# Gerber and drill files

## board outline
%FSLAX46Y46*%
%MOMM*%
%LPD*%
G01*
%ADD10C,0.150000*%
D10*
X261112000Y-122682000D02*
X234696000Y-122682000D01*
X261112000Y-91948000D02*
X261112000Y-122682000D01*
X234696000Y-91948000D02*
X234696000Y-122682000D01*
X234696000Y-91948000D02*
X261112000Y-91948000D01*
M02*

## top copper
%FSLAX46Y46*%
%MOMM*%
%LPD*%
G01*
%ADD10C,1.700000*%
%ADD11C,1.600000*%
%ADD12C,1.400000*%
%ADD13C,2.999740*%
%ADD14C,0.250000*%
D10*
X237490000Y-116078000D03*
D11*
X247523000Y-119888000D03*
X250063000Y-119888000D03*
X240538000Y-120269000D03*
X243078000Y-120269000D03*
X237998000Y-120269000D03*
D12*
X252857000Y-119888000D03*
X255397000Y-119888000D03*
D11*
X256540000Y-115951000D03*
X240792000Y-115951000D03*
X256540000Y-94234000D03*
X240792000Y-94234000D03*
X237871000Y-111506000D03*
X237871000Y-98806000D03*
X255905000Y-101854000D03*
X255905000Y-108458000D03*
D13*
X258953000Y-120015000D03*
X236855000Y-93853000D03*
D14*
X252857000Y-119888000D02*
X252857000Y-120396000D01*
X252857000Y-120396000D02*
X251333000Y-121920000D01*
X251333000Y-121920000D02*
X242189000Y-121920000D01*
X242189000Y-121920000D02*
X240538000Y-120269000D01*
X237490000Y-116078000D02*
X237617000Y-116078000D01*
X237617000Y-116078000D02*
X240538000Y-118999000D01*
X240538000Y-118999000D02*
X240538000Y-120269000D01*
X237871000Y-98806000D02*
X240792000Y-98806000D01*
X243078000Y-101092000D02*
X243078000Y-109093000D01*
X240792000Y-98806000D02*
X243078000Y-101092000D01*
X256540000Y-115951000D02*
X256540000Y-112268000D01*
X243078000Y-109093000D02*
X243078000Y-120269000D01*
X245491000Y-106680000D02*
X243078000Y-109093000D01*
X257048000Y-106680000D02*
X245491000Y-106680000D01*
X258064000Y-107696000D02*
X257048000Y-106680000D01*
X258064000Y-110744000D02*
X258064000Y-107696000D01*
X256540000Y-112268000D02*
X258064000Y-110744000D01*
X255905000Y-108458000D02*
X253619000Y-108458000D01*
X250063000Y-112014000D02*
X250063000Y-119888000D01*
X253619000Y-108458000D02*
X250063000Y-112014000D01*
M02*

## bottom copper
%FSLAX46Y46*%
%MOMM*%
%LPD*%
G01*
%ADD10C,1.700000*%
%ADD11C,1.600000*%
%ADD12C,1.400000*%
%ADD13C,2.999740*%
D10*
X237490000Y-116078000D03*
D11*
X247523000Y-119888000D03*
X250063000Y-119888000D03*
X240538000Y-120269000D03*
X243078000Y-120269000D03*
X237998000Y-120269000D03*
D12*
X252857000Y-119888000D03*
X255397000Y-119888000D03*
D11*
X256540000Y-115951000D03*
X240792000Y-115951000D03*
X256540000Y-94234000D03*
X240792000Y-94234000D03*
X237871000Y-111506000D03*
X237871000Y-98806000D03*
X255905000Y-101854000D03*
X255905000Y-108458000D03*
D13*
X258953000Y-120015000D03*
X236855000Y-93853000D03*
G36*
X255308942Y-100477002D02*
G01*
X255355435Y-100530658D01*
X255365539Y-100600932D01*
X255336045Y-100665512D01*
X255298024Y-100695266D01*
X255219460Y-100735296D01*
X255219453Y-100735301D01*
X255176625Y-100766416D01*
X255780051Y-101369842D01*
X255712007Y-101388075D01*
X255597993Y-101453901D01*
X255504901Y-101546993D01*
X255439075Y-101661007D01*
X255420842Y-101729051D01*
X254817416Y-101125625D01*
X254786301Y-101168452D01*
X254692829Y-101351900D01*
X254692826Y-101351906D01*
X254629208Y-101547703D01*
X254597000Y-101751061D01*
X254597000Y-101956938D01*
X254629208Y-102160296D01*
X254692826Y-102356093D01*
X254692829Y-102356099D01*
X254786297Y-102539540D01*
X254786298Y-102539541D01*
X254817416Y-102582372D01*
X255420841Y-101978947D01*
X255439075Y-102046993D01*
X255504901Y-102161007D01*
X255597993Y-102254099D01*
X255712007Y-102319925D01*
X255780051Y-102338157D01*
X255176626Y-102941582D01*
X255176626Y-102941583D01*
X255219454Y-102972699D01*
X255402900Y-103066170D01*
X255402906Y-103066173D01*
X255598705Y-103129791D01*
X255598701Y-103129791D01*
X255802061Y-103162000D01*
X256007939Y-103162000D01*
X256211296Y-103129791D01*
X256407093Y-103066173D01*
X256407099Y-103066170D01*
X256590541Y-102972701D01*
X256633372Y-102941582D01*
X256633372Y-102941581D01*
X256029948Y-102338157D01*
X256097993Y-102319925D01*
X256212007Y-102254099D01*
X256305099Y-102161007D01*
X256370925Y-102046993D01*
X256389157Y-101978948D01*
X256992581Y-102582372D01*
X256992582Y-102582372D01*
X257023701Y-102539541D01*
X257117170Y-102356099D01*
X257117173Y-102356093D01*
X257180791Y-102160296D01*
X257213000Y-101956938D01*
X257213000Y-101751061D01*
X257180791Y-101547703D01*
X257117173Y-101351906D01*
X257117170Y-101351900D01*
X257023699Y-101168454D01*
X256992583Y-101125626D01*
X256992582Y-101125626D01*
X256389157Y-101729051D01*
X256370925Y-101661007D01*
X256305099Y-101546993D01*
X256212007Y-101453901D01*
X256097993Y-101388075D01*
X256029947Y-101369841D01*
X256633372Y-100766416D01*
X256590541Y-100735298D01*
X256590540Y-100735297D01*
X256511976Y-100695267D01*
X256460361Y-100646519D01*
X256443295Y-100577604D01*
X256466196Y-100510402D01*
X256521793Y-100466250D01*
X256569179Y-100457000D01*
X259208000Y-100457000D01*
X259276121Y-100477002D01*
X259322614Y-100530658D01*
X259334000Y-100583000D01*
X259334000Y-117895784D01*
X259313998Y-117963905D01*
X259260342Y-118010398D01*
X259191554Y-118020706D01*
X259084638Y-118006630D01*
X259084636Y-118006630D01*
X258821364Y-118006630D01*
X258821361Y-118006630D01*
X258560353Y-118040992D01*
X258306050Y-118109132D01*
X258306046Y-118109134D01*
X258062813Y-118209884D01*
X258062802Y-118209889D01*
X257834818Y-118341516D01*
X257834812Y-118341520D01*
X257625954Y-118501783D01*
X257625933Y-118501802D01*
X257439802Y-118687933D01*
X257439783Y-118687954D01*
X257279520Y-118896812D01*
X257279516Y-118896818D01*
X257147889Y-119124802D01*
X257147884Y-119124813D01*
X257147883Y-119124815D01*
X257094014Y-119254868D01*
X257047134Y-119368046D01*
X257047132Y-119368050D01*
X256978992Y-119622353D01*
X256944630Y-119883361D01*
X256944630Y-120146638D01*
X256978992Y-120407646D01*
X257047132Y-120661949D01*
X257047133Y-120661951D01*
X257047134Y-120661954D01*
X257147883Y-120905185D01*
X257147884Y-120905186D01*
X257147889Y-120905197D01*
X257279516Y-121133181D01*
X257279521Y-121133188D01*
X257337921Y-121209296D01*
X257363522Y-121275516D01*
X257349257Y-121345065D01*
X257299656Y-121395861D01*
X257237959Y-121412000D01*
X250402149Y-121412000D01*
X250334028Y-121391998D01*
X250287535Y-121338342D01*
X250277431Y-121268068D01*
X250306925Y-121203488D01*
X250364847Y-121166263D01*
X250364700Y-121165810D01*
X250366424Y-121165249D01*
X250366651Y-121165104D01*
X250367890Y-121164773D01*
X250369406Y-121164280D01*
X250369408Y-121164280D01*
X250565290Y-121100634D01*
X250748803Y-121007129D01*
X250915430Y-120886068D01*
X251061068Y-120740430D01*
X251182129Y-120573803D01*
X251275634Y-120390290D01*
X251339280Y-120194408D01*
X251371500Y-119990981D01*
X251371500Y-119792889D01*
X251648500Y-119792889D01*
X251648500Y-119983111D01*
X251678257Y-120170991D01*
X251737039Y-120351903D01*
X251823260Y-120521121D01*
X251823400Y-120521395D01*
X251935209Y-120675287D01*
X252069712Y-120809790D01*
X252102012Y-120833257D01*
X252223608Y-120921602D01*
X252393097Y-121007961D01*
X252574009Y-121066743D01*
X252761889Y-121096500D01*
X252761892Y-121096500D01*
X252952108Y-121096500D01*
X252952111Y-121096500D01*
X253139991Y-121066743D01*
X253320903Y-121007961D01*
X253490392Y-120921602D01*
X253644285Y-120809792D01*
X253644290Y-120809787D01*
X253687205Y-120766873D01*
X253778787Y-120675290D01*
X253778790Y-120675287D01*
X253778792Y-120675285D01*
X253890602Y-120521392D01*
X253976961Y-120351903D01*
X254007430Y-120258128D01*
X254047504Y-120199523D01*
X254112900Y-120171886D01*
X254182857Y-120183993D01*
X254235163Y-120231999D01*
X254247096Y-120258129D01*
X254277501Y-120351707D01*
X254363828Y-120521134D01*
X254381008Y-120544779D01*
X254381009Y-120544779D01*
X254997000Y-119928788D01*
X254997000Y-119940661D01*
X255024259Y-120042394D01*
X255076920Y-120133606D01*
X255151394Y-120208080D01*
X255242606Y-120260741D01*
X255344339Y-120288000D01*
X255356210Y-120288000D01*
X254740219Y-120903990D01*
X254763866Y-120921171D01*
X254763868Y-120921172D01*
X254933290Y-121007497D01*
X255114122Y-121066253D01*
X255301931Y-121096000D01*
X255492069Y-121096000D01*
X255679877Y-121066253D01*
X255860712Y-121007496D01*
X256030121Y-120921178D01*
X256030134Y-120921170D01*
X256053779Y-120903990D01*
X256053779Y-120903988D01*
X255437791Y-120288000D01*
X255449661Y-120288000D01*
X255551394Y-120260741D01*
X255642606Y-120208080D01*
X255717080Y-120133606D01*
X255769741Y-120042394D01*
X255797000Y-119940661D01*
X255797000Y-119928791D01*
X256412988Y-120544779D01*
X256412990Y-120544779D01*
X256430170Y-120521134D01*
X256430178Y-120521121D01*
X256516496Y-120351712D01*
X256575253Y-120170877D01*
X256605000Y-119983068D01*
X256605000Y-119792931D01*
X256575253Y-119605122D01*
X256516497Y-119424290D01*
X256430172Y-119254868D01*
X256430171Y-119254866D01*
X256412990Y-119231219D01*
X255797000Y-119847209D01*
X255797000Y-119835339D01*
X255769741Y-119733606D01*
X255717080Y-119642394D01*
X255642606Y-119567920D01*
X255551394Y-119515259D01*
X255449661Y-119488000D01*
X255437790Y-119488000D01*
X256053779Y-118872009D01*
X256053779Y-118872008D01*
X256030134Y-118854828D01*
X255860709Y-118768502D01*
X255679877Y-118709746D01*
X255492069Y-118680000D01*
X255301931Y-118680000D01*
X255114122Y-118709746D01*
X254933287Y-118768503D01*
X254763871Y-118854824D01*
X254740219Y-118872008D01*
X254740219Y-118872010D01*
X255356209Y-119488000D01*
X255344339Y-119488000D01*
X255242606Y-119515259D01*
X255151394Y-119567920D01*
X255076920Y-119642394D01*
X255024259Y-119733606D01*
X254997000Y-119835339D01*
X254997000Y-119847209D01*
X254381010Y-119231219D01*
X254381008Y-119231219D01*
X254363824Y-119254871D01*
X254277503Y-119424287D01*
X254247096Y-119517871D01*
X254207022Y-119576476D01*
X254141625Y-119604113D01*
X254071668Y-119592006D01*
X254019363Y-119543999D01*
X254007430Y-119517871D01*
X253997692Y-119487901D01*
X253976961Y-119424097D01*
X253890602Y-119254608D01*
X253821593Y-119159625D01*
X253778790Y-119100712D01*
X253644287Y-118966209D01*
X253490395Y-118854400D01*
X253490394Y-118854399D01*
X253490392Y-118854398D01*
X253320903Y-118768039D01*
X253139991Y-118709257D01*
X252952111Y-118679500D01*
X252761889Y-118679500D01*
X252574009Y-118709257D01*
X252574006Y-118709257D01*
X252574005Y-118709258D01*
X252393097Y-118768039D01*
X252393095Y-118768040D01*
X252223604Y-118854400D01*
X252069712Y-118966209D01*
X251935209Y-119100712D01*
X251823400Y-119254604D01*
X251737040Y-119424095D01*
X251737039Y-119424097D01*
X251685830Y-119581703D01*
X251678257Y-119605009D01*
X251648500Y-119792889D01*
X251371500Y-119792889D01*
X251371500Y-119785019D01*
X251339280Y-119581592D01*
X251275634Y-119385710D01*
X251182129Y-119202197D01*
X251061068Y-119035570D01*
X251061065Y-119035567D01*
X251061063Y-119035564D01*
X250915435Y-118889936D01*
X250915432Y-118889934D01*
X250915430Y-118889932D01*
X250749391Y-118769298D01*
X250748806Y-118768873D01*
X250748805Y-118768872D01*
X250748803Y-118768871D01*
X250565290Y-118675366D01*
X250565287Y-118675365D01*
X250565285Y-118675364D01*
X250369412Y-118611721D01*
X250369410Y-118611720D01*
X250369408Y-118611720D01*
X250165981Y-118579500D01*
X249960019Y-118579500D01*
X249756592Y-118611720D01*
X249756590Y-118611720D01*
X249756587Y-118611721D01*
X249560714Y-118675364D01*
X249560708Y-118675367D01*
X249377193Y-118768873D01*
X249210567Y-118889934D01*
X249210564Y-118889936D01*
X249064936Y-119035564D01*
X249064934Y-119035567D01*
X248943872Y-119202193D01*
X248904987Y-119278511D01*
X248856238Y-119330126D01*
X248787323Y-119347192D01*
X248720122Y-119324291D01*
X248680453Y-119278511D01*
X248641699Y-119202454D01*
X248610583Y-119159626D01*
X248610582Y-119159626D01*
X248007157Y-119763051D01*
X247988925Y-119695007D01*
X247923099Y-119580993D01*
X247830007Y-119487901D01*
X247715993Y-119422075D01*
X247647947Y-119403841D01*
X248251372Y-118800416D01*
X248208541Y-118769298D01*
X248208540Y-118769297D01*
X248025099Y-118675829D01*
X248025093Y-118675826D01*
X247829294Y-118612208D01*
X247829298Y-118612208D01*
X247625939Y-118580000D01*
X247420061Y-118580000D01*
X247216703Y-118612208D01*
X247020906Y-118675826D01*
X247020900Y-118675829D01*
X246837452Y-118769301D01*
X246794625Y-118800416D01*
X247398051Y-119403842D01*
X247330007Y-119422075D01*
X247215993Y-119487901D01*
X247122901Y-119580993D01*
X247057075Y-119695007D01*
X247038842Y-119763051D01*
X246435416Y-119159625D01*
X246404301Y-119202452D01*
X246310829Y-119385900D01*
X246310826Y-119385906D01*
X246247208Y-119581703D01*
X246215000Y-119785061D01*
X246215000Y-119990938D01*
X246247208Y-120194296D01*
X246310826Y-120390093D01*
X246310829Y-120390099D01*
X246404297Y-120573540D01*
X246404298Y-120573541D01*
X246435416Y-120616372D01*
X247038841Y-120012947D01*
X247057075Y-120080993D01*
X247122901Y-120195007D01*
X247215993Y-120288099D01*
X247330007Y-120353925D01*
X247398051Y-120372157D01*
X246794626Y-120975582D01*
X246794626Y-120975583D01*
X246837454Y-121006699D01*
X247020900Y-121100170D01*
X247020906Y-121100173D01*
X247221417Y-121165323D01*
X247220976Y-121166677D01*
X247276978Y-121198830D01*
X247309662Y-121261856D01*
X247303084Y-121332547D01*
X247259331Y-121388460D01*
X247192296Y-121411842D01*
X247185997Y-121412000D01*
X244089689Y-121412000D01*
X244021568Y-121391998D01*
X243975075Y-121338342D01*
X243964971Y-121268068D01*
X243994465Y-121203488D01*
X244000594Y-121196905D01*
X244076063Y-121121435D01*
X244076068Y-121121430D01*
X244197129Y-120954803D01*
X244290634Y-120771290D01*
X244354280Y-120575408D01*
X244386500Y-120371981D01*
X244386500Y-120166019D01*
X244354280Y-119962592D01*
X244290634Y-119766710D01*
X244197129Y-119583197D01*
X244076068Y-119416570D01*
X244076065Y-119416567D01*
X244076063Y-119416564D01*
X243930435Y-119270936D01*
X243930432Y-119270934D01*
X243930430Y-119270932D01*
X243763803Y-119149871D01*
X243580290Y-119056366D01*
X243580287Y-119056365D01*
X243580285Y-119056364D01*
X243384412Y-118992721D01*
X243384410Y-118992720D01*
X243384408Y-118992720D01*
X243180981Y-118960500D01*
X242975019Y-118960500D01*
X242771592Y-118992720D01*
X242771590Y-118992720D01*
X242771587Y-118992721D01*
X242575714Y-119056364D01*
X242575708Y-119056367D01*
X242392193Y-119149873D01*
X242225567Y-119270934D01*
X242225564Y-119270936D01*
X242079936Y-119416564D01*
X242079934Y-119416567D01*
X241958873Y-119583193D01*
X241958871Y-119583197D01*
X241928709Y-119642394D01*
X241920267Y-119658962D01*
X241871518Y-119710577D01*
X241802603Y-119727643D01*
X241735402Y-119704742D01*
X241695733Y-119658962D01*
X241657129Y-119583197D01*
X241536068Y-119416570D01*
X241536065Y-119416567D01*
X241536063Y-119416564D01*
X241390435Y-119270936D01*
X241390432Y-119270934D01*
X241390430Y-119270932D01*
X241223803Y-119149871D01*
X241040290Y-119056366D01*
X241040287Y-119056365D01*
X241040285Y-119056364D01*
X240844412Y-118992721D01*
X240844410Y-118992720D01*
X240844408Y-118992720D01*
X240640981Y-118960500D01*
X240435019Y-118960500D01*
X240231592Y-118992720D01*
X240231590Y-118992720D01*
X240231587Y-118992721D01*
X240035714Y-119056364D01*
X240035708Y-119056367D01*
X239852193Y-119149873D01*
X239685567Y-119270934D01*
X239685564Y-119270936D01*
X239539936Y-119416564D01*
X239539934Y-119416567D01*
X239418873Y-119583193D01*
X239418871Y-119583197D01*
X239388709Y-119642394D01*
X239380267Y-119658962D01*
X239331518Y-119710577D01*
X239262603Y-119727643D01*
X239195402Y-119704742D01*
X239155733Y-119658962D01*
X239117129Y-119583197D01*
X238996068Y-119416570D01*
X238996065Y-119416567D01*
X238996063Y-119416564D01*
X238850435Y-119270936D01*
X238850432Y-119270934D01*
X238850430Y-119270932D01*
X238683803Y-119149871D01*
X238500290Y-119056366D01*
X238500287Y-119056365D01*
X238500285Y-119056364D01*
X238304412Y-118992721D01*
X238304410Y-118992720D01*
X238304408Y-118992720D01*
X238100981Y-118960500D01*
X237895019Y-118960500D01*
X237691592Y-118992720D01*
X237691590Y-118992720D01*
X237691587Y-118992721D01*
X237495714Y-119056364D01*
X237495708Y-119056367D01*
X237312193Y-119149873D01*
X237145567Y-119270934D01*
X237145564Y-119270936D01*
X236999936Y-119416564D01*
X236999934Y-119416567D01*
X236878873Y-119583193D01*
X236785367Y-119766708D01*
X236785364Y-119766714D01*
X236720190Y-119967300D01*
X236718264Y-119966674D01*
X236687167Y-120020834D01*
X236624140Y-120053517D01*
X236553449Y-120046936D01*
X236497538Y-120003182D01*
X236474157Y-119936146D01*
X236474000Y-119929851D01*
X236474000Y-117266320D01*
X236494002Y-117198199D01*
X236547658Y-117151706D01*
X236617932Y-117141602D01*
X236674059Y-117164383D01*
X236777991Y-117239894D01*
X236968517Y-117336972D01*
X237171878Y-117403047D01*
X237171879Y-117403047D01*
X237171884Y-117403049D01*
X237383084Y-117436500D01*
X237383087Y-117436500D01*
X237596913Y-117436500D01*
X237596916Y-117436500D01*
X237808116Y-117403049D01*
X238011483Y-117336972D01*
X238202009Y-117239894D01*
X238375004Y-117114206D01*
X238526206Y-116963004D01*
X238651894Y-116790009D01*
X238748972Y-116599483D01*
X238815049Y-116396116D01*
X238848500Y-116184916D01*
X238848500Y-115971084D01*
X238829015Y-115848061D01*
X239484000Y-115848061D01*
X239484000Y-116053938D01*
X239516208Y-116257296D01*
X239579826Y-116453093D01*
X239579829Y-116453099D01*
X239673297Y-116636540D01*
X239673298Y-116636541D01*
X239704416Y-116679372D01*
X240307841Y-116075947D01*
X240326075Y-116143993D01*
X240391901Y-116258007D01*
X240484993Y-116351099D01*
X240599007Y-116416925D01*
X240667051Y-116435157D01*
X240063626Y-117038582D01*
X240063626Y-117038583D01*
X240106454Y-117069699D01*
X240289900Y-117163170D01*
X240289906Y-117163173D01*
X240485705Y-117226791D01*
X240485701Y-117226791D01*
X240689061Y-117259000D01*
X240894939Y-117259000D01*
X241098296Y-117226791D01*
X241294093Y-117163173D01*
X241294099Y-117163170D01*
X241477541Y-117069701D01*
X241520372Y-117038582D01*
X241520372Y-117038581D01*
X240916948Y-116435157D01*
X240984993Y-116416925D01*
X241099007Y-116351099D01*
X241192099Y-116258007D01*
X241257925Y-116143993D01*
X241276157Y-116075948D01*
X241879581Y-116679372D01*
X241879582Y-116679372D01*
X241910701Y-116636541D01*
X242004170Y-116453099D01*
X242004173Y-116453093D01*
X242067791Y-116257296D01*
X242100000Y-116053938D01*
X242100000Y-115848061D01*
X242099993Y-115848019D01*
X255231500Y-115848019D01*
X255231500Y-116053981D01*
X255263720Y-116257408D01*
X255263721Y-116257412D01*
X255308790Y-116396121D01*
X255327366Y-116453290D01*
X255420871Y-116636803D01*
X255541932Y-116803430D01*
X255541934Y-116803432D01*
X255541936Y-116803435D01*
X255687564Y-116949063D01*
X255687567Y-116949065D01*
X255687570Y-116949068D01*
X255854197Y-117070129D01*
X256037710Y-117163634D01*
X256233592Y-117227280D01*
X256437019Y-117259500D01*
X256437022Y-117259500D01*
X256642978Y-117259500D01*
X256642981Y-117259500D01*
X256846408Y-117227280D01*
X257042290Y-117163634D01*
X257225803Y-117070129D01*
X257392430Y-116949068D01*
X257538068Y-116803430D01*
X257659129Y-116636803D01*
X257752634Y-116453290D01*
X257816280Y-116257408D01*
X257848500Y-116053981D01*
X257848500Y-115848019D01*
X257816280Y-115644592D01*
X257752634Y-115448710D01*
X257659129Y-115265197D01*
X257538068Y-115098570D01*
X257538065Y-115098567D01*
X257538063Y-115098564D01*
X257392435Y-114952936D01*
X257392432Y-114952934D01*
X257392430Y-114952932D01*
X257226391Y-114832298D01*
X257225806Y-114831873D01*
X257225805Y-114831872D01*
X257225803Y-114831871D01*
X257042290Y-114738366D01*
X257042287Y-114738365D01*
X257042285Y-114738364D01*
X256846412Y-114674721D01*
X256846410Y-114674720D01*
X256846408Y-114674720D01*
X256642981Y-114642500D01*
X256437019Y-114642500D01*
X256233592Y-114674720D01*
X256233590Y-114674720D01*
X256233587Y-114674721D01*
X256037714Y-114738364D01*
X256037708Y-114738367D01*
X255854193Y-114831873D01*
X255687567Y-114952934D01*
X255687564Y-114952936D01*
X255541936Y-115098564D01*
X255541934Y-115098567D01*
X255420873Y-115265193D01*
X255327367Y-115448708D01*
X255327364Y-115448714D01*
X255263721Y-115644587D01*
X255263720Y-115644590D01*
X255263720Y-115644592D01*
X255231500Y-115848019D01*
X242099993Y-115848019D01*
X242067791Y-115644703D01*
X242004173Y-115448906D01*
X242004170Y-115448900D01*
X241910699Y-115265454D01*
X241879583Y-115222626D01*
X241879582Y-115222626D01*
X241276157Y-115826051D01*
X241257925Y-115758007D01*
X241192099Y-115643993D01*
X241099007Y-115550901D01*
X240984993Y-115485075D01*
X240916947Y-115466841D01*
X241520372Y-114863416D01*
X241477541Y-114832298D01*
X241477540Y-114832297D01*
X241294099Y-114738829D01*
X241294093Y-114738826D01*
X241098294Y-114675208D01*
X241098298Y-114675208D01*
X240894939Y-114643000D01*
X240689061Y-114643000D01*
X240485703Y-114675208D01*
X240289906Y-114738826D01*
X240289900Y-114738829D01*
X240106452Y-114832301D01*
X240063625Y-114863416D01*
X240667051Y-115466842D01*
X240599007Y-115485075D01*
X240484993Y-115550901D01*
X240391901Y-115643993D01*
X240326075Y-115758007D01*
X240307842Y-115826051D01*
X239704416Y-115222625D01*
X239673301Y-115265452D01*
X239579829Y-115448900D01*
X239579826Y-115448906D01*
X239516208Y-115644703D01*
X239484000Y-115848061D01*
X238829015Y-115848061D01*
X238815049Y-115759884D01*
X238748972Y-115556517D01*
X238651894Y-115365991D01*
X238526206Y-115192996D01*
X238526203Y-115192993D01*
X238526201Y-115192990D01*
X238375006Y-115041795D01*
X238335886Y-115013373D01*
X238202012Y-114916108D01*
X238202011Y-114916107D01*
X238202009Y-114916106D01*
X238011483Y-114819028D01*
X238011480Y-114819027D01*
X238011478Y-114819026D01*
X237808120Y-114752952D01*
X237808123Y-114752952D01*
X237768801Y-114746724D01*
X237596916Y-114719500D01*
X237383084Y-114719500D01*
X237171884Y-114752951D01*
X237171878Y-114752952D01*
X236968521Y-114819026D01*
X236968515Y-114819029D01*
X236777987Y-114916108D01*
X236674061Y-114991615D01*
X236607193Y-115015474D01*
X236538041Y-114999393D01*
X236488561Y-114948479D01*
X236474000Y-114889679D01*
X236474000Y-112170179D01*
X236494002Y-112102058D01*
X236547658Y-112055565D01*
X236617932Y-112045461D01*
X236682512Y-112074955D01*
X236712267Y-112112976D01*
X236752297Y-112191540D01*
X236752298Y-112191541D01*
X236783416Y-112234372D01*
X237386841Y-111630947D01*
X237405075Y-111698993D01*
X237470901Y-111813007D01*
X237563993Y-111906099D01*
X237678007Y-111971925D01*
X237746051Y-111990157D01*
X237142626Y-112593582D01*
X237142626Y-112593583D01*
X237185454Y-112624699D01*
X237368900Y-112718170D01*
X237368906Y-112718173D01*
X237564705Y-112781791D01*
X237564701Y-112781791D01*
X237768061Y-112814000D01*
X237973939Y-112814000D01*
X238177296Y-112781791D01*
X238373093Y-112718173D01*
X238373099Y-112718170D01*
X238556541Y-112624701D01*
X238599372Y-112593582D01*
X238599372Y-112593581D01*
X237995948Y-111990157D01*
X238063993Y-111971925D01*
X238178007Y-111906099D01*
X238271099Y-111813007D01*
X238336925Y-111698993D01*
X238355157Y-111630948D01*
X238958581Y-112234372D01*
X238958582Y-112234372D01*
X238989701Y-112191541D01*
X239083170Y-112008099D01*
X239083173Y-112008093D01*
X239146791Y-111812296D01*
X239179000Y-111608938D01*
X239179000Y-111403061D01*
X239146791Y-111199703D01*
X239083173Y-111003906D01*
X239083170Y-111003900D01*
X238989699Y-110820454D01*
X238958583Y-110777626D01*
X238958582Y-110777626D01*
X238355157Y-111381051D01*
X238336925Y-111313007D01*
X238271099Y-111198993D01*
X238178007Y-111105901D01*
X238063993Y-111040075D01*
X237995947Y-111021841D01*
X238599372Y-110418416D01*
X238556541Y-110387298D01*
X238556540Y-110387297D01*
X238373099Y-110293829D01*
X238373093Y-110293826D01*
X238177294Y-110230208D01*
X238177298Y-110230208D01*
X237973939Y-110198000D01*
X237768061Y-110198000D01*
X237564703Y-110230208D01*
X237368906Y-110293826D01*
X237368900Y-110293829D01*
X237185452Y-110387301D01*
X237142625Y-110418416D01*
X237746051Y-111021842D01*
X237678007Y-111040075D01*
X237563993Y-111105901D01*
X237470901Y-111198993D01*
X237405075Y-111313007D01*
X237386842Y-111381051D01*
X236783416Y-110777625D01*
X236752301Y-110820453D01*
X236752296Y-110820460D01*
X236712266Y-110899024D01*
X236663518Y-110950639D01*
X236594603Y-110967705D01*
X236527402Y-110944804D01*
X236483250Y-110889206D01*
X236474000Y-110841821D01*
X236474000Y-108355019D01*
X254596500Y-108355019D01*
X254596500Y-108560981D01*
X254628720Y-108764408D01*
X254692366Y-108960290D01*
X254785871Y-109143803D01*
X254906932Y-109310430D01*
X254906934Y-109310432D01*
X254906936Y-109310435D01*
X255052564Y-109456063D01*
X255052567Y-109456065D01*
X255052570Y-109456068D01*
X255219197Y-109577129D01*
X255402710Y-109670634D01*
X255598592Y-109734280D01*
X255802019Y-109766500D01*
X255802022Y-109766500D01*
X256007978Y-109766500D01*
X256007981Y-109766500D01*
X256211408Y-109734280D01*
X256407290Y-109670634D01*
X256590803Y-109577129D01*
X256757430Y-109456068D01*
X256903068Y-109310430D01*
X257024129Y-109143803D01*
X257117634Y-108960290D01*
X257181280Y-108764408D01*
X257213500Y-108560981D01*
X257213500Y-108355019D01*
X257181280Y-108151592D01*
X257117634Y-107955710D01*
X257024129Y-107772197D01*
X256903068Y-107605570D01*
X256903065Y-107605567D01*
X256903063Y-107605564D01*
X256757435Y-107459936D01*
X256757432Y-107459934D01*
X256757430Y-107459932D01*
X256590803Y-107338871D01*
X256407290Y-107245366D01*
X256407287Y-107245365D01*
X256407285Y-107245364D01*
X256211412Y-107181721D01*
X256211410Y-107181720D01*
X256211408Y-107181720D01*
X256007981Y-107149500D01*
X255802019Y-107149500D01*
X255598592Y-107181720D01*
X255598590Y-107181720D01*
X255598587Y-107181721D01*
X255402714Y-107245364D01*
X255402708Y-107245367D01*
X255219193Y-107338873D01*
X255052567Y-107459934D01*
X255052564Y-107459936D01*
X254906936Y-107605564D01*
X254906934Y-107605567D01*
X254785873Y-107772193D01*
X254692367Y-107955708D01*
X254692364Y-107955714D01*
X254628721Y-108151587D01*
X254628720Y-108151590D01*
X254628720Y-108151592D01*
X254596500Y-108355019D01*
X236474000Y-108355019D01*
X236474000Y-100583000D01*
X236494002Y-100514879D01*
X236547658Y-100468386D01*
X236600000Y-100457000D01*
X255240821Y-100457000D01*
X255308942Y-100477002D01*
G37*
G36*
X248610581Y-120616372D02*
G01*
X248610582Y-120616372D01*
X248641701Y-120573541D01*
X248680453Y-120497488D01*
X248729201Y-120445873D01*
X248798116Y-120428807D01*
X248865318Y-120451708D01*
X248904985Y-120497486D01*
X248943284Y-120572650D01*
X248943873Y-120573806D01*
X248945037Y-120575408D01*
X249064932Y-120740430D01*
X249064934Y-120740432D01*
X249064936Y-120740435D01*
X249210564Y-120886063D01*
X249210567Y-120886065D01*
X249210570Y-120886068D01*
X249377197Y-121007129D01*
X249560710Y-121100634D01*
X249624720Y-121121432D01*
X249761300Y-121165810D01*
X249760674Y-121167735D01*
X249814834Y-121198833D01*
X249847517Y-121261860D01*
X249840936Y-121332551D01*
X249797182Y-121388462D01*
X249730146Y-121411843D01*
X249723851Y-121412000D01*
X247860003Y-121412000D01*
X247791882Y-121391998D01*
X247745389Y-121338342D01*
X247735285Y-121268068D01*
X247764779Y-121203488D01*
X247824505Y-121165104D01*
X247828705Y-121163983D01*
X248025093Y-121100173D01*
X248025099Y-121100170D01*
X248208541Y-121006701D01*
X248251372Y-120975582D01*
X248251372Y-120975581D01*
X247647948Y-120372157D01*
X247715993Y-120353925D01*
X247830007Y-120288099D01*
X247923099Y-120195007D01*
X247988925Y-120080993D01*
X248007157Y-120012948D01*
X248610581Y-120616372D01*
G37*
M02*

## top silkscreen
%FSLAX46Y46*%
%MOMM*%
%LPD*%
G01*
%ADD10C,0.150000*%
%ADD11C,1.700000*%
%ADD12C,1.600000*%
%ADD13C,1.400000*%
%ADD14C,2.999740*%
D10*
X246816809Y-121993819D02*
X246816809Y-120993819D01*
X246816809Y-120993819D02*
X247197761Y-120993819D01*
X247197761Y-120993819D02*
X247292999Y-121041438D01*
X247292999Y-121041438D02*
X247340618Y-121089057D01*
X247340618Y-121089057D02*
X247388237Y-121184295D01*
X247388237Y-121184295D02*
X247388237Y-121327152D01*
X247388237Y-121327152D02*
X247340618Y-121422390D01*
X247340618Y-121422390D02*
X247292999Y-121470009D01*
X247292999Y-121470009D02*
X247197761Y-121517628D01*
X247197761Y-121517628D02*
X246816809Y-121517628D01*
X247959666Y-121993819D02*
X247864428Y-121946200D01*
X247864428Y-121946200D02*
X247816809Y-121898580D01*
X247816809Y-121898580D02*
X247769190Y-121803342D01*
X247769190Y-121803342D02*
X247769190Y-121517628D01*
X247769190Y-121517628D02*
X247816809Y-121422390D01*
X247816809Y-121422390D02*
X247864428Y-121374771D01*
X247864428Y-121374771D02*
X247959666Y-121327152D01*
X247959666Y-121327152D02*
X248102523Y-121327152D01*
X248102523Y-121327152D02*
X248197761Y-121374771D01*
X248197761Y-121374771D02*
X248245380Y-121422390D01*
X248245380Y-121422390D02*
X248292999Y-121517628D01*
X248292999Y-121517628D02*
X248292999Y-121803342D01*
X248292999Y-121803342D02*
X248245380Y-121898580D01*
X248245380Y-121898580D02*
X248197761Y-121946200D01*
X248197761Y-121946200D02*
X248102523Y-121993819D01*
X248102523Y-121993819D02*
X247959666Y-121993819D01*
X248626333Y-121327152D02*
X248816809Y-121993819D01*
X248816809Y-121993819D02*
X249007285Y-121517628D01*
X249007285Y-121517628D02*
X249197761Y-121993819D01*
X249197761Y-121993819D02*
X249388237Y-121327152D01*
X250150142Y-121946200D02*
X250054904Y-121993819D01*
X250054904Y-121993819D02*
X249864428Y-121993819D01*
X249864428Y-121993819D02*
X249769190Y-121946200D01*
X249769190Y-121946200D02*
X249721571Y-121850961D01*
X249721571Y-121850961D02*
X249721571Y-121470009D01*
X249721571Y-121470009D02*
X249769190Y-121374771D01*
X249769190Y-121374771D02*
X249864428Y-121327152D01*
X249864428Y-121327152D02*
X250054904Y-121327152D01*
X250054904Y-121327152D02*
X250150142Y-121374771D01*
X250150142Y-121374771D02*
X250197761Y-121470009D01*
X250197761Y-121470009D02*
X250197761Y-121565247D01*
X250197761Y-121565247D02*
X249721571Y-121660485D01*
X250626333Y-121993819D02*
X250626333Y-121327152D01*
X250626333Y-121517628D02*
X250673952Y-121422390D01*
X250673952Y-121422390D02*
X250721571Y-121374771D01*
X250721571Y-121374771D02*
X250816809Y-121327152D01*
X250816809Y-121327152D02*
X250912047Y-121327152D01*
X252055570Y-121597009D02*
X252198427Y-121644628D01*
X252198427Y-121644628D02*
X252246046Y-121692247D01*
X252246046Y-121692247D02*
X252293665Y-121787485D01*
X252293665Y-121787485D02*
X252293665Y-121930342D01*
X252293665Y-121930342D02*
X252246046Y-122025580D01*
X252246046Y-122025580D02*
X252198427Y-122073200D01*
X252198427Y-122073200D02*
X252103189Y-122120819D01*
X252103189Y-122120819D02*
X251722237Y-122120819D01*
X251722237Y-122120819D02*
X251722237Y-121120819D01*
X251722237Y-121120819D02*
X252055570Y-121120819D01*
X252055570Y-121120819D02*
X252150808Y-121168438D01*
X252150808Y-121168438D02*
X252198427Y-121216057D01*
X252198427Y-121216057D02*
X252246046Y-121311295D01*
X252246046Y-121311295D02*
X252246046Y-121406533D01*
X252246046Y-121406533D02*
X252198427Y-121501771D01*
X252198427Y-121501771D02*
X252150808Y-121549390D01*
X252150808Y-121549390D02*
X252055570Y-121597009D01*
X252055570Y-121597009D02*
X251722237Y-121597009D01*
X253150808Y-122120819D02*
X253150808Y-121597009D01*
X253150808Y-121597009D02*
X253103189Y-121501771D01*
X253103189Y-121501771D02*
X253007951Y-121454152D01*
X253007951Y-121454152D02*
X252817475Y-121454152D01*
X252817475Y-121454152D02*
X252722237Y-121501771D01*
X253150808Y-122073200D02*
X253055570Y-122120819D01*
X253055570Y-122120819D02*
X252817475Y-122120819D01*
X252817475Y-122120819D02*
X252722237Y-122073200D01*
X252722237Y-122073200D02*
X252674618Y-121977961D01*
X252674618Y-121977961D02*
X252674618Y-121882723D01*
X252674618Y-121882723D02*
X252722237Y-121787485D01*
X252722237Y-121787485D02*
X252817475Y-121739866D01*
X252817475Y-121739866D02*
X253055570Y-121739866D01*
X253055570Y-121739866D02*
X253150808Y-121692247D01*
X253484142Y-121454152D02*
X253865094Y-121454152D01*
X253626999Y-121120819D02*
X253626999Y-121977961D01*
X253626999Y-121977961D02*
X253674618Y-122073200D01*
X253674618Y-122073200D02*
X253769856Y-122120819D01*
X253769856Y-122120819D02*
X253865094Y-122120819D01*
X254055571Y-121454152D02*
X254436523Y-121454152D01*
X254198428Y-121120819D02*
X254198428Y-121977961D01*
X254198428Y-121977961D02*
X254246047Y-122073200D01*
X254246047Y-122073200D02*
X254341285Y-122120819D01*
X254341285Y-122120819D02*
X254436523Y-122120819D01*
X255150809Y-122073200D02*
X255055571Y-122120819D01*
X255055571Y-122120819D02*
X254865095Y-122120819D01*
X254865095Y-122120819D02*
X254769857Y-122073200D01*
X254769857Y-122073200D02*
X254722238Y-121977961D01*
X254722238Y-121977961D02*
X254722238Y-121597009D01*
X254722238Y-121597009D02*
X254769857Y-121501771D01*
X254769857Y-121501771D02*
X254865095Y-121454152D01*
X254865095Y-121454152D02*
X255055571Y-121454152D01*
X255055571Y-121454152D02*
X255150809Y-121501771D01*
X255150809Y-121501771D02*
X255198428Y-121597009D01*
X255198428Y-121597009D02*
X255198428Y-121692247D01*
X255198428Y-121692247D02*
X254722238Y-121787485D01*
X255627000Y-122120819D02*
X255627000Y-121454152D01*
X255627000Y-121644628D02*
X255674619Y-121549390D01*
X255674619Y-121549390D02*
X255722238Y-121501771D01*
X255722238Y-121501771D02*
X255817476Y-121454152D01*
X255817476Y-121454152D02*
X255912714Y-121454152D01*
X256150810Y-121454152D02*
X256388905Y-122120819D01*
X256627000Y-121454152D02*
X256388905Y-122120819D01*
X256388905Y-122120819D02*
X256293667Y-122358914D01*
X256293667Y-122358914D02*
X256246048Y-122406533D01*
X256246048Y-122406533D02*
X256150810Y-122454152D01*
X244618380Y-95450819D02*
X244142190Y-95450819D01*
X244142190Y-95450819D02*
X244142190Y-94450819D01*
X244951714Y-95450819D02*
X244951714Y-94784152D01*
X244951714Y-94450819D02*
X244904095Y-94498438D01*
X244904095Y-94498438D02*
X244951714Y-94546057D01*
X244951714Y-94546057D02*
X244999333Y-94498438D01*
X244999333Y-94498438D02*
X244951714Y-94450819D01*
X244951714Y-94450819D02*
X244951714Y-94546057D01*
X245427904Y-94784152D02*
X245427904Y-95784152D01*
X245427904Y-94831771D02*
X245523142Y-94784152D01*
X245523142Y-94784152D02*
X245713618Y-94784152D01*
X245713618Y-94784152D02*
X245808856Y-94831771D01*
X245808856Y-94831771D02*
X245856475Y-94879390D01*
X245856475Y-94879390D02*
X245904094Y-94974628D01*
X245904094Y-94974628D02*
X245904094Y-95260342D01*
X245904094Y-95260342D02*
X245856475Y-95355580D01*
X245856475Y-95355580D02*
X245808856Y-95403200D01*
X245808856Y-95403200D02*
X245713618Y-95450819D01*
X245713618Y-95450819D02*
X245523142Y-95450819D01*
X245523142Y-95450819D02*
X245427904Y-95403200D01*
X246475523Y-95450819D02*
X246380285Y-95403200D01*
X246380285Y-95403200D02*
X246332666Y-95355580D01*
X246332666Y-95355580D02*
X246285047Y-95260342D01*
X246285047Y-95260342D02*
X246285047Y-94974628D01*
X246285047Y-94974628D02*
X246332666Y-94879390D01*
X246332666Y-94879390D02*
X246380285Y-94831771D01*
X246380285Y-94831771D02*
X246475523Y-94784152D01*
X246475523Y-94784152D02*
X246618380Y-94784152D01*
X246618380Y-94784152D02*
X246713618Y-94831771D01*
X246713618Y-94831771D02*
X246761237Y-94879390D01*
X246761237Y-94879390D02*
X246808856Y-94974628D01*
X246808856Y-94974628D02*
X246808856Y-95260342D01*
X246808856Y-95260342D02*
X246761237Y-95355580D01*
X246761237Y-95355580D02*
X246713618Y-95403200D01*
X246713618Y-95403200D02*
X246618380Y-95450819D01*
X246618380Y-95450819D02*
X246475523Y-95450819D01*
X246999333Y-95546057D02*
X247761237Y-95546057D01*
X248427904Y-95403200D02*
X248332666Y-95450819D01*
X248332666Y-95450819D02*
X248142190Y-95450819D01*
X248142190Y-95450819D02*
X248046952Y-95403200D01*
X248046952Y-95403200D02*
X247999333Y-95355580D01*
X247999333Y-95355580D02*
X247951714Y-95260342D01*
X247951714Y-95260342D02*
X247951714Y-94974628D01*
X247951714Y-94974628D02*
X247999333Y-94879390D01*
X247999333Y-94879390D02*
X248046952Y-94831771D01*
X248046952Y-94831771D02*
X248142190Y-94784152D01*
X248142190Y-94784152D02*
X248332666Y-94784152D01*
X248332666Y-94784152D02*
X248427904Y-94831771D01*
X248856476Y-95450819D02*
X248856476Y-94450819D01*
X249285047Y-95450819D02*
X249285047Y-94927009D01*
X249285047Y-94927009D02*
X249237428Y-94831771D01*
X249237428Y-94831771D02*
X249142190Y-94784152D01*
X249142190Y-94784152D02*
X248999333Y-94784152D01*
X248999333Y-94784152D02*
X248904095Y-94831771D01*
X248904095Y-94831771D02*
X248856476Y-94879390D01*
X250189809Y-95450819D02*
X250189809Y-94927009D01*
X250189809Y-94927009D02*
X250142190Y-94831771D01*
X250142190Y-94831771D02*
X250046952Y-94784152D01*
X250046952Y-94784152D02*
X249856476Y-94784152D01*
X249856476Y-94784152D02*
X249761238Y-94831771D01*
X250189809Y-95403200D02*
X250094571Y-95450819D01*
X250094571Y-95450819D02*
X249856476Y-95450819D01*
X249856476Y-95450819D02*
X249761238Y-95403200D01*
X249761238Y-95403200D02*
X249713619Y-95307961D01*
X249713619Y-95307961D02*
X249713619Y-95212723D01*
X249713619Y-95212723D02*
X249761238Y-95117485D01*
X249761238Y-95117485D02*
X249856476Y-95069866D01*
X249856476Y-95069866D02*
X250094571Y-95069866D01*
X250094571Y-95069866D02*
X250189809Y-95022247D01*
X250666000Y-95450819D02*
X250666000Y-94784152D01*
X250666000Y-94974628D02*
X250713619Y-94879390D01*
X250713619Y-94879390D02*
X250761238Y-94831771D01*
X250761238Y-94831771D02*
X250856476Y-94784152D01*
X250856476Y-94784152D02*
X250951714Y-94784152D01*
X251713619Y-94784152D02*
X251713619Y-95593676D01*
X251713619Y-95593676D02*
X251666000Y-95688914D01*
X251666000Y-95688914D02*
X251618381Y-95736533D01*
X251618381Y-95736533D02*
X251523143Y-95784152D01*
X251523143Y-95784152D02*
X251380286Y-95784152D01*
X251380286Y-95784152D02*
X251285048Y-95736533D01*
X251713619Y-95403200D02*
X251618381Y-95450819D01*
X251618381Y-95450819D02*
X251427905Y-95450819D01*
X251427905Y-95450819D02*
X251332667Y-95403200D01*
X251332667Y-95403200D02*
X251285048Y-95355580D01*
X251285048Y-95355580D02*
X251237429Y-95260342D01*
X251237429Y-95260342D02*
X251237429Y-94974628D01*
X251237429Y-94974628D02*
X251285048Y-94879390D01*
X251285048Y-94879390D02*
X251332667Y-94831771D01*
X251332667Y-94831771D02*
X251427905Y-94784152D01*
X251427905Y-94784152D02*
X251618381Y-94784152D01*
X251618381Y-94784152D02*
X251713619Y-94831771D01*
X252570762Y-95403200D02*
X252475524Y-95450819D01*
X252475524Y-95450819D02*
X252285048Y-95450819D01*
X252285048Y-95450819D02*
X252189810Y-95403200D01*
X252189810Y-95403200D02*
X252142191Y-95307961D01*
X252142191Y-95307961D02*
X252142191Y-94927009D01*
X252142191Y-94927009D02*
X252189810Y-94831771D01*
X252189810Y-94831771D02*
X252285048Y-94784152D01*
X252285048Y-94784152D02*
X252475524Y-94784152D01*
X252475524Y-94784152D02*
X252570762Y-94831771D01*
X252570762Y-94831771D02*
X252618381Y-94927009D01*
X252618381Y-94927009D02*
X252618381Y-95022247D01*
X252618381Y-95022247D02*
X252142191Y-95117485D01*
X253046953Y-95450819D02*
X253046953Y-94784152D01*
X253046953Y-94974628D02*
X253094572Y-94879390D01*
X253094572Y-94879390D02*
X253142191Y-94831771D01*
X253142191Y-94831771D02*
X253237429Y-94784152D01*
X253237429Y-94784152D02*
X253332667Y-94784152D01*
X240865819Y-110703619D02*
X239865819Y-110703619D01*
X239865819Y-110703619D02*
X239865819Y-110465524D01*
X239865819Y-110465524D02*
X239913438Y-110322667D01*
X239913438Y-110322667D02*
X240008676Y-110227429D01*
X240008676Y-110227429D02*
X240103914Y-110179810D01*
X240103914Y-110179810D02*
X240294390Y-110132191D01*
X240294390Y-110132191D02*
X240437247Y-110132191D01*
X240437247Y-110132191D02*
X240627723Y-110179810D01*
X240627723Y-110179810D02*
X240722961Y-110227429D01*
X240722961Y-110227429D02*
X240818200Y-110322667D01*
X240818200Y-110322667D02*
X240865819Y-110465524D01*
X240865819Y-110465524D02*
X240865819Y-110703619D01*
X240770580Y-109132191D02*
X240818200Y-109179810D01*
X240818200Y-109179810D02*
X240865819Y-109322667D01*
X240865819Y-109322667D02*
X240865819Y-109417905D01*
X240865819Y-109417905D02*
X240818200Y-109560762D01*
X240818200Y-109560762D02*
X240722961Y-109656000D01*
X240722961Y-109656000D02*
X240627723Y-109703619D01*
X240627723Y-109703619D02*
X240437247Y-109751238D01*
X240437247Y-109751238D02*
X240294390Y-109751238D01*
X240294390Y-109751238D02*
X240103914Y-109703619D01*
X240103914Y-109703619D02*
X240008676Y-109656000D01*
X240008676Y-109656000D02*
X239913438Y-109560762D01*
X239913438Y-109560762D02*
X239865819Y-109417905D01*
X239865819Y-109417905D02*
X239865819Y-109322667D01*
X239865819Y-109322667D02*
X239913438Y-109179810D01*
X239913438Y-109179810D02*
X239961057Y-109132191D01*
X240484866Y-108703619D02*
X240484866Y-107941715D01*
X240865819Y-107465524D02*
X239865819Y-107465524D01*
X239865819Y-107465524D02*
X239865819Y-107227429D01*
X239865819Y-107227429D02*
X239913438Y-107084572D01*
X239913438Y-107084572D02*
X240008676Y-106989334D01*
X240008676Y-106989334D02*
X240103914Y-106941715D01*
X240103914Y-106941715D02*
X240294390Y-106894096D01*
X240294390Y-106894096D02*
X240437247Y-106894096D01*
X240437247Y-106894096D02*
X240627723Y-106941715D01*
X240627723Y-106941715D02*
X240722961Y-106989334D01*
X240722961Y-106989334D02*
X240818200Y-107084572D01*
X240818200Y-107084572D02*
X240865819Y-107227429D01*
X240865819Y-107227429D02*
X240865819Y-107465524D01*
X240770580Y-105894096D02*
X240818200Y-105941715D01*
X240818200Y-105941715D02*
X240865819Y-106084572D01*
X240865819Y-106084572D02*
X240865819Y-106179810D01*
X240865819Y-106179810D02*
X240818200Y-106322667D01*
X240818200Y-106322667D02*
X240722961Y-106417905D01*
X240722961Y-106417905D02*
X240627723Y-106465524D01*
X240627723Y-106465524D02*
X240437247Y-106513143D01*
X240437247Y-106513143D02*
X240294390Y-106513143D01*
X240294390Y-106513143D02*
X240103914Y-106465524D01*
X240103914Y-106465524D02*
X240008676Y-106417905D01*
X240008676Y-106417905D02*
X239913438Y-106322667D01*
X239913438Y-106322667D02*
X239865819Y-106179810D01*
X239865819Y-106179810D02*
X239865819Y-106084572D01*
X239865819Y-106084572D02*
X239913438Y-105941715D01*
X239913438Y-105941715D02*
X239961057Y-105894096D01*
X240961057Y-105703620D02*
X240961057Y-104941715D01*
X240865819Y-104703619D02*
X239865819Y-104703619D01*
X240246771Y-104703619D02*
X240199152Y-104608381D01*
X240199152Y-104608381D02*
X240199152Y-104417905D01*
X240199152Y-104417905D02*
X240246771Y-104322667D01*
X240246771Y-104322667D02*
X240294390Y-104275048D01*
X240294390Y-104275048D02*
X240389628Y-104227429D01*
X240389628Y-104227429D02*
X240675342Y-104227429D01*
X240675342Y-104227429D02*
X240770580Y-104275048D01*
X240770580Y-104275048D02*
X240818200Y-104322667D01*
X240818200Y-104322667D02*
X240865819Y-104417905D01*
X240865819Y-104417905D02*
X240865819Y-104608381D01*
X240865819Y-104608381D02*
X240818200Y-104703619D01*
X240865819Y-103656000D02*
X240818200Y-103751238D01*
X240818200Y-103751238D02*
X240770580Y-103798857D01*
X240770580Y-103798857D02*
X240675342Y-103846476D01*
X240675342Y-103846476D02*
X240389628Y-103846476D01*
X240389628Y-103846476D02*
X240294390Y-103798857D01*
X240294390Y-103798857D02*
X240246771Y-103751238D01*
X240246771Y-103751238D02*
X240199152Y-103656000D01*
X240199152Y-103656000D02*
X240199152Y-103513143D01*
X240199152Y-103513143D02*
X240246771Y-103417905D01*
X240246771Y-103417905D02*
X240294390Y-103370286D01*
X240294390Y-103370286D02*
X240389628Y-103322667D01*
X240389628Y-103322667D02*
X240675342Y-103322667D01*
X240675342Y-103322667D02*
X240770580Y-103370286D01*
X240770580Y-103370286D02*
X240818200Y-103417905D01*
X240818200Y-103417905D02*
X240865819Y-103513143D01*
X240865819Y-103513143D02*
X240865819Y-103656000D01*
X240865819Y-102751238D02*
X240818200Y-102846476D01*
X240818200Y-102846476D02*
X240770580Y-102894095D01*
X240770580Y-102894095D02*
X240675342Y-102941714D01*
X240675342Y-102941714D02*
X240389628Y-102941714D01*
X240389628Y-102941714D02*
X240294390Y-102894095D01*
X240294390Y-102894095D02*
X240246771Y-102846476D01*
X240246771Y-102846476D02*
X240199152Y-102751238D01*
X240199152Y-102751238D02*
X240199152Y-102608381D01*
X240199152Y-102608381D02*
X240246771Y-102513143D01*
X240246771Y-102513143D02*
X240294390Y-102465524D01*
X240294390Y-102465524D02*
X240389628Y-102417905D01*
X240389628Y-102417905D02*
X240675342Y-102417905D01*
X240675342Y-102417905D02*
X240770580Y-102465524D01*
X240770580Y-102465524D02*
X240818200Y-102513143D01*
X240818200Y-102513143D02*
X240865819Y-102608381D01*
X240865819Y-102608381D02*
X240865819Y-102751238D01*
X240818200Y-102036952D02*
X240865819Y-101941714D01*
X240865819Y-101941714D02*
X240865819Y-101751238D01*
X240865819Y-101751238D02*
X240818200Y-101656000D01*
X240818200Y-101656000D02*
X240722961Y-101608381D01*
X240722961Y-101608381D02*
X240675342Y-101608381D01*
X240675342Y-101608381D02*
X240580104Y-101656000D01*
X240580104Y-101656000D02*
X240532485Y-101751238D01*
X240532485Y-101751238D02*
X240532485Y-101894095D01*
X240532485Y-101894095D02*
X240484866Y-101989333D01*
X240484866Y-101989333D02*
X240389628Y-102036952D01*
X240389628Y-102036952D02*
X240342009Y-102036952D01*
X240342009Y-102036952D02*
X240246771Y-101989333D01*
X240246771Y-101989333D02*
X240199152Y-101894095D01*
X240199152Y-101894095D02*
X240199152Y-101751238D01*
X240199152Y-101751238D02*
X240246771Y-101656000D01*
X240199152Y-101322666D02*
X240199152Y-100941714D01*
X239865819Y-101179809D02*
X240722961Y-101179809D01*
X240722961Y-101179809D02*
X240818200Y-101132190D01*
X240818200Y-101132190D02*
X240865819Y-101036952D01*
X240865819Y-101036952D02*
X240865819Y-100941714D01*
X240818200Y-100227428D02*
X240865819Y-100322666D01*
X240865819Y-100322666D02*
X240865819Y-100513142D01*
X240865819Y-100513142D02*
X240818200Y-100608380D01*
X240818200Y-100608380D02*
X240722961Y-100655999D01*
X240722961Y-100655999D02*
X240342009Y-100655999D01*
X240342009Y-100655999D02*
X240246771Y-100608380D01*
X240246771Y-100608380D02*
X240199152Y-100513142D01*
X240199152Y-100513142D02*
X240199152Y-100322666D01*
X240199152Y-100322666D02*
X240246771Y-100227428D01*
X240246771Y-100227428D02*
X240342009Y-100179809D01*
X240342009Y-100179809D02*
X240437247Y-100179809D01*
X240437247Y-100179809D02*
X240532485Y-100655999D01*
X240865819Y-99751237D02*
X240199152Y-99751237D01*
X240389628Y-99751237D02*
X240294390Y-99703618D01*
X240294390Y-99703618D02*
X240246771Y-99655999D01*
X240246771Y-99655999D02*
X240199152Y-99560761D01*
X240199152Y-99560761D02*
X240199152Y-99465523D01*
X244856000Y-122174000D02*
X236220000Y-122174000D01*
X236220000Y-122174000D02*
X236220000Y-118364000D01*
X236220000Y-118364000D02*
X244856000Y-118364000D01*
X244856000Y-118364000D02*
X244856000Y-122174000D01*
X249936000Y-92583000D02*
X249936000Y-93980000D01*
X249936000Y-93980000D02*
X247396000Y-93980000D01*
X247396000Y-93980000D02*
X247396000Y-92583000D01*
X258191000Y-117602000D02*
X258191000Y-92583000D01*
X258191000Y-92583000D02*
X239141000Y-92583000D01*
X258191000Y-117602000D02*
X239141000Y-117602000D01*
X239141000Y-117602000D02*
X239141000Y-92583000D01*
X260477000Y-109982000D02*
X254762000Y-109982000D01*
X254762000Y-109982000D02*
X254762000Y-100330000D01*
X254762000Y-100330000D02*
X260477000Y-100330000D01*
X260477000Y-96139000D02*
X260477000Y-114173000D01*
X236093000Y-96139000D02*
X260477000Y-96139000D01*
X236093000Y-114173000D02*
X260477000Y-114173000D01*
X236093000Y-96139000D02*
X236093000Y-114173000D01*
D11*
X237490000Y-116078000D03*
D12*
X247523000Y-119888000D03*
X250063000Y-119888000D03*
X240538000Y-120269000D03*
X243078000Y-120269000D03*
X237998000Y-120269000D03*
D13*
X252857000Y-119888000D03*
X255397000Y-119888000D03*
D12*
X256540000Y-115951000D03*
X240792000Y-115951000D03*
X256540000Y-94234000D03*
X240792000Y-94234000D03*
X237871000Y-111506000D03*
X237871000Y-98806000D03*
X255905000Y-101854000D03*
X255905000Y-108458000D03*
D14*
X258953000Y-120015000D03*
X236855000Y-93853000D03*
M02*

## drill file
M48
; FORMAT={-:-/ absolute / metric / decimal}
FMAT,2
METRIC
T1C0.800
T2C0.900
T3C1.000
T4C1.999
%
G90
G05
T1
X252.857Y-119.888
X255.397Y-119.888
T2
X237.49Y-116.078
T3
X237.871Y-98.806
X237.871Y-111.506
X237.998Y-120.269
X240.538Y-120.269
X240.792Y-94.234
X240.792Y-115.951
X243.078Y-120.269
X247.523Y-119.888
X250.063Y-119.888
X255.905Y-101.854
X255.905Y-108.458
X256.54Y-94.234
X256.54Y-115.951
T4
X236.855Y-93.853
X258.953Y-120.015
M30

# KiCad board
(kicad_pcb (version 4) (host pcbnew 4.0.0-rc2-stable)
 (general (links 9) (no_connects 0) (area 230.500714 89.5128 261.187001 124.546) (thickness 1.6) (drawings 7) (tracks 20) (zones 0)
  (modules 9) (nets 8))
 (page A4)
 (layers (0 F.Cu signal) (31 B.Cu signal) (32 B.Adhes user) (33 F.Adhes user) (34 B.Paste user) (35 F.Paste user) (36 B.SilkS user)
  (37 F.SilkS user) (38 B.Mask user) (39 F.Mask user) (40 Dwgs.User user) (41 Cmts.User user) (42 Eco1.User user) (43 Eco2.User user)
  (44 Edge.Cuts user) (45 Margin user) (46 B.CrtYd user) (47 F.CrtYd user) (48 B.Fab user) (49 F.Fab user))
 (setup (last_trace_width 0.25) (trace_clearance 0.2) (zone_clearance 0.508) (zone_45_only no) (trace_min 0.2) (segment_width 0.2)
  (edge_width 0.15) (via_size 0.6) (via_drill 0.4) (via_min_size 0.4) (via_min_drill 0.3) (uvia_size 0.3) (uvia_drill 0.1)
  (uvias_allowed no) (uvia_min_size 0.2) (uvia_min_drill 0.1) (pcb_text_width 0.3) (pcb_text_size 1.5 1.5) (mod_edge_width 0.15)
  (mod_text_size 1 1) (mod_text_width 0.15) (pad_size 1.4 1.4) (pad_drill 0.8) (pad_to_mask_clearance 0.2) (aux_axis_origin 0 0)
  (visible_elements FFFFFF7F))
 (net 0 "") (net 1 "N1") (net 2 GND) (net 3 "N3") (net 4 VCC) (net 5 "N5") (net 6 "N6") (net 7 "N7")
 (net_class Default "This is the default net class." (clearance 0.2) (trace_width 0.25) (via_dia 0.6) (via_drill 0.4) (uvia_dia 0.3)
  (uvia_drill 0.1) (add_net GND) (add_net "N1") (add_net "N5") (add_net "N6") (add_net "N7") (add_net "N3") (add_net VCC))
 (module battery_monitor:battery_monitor (layer F.Cu) (at 237.49 116.078)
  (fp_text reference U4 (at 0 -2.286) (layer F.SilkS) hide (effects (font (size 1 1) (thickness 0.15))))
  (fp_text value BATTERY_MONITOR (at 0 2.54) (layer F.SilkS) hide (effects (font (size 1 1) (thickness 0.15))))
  (pad 1 thru_hole circle (at 0 0) (size 1.7 1.7) (drill 0.9) (layers *.Cu *.Mask F.SilkS) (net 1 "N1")))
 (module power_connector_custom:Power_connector (layer F.Cu) (at 248.793 119.888)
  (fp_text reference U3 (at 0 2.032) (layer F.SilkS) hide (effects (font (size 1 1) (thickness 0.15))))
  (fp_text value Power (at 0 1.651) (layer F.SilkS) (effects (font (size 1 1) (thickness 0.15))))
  (pad 1 thru_hole circle (at -1.27 0) (size 1.6 1.6) (drill 1) (layers *.Cu *.Mask F.SilkS) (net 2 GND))
  (pad 2 thru_hole circle (at 1.27 0) (size 1.6 1.6) (drill 1) (layers *.Cu *.Mask F.SilkS) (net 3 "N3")))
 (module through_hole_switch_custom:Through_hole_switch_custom (layer F.Cu) (at 240.538 120.269 180)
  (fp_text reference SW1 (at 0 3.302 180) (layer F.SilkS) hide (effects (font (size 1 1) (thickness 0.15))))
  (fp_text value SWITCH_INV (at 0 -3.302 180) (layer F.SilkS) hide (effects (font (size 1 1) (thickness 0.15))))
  (fp_line (start -4.318 -1.905) (end 4.318 -1.905) (layer F.SilkS) (width 0.15))
  (fp_line (start 4.318 -1.905) (end 4.318 1.905) (layer F.SilkS) (width 0.15))
  (fp_line (start 4.318 1.905) (end -4.318 1.905) (layer F.SilkS) (width 0.15))
  (fp_line (start -4.318 1.905) (end -4.318 -1.905) (layer F.SilkS) (width 0.15))
  (pad 2 thru_hole circle (at 0 0 180) (size 1.6 1.6) (drill 1) (layers *.Cu *.Mask F.SilkS) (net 1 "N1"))
  (pad 1 thru_hole circle (at -2.54 0 180) (size 1.6 1.6) (drill 1) (layers *.Cu *.Mask F.SilkS) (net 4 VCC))
  (pad 3 thru_hole circle (at 2.54 0 180) (size 1.6 1.6) (drill 1) (layers *.Cu *.Mask F.SilkS) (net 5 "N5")))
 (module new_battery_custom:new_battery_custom (layer F.Cu) (at 254.127 119.888)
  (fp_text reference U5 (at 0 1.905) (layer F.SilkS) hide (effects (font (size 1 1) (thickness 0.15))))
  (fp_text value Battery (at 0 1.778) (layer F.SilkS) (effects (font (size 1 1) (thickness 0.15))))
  (pad 2 thru_hole circle (at -1.27 0) (size 1.4 1.4) (drill 0.8) (layers *.Cu *.Mask F.SilkS) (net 1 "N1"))
  (pad 1 thru_hole circle (at 1.27 0) (size 1.4 1.4) (drill 0.8) (layers *.Cu *.Mask F.SilkS) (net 2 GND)))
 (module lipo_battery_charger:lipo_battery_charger (layer F.Cu) (at 248.666 105.156 180) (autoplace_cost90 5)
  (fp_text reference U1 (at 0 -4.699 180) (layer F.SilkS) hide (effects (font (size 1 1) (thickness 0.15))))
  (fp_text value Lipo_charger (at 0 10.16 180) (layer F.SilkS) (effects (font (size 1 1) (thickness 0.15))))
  (fp_line (start -1.27 12.573) (end -1.27 11.176) (layer F.SilkS) (width 0.15))
  (fp_line (start -1.27 11.176) (end 1.27 11.176) (layer F.SilkS) (width 0.15))
  (fp_line (start 1.27 11.176) (end 1.27 12.573) (layer F.SilkS) (width 0.15))
  (fp_line (start -9.525 -12.446) (end -9.525 12.573) (layer F.SilkS) (width 0.15))
  (fp_line (start -9.525 12.573) (end 9.525 12.573) (layer F.SilkS) (width 0.15))
  (fp_line (start -9.525 -12.446) (end 9.525 -12.446) (layer F.SilkS) (width 0.15))
  (fp_line (start 9.525 -12.446) (end 9.525 12.573) (layer F.SilkS) (width 0.15))
  (pad 2 thru_hole circle (at -7.874 -10.795 180) (size 1.6 1.6) (drill 1) (layers *.Cu *.Mask F.SilkS) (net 4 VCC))
  (pad 1 thru_hole circle (at 7.874 -10.795 180) (size 1.6 1.6) (drill 1) (layers *.Cu *.Mask F.SilkS) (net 2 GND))
  (pad 3 thru_hole circle (at -7.874 10.922 180) (size 1.6 1.6) (drill 1) (layers *.Cu *.Mask F.SilkS) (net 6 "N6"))
  (pad 4 thru_hole circle (at 7.874 10.922 180) (size 1.6 1.6) (drill 1) (layers *.Cu *.Mask F.SilkS) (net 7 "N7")))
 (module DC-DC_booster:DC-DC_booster (layer F.Cu) (at 248.158 105.156 90)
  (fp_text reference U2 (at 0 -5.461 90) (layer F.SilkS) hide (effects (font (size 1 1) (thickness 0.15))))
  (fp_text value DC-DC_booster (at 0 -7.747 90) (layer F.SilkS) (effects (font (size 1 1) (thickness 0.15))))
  (fp_line (start -4.826 12.319) (end -4.826 6.604) (layer F.SilkS) (width 0.15))
  (fp_line (start -4.826 6.604) (end 4.826 6.604) (layer F.SilkS) (width 0.15))
  (fp_line (start 4.826 6.604) (end 4.826 12.319) (layer F.SilkS) (width 0.15))
  (fp_line (start 9.017 12.319) (end -9.017 12.319) (layer F.SilkS) (width 0.15))
  (fp_line (start 9.017 -12.065) (end 9.017 12.319) (layer F.SilkS) (width 0.15))
  (fp_line (start -9.017 -12.065) (end -9.017 12.319) (layer F.SilkS) (width 0.15))
  (fp_line (start 9.017 -12.065) (end -9.017 -12.065) (layer F.SilkS) (width 0.15))
  (pad 1 thru_hole circle (at -6.35 -10.287 90) (size 1.6 1.6) (drill 1) (layers *.Cu *.Mask F.SilkS) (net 2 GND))
  (pad 2 thru_hole circle (at 6.35 -10.287 90) (size 1.6 1.6) (drill 1) (layers *.Cu *.Mask F.SilkS) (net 4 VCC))
  (pad 3 thru_hole circle (at 3.302 7.747 90) (size 1.6 1.6) (drill 1) (layers *.Cu *.Mask F.SilkS) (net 2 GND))
  (pad 4 thru_hole circle (at -3.302 7.747 90) (size 1.6 1.6) (drill 1) (layers *.Cu *.Mask F.SilkS) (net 3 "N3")))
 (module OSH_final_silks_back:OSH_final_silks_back (layer F.Cu) (at 248.793 114.427)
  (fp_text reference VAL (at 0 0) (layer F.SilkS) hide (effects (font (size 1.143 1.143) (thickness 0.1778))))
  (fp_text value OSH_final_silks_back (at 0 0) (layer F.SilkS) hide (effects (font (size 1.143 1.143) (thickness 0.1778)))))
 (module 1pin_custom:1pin (layer F.Cu) (at 258.953 120.015)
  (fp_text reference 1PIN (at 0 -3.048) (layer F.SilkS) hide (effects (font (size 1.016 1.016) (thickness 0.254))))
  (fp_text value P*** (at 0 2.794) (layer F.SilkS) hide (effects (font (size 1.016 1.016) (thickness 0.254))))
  (pad 1 thru_hole circle (at 0 0) (size 2.99974 2.99974) (drill 1.99898) (layers *.Cu *.Mask F.SilkS)))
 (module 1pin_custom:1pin (layer F.Cu) (at 236.855 93.853)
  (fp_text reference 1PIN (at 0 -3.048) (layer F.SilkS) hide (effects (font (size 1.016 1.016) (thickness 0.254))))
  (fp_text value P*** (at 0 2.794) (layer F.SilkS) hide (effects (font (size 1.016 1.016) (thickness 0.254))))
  (pad 1 thru_hole circle (at 0 0) (size 2.99974 2.99974) (drill 1.99898) (layers *.Cu *.Mask F.SilkS)))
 (gr_line (start 261.112 122.682) (end 234.696 122.682) (angle 90) (layer Edge.Cuts) (width 0.15))
 (gr_line (start 261.112 91.948) (end 261.112 122.682) (angle 90) (layer Edge.Cuts) (width 0.15))
 (gr_line (start 234.696 91.948) (end 234.696 122.682) (angle 90) (layer Edge.Cuts) (width 0.15))
 (gr_line (start 234.696 91.948) (end 261.112 91.948) (angle 90) (layer Edge.Cuts) (width 0.15))
 (segment (start 252.857 119.888) (end 252.857 120.396) (width 0.25) (layer F.Cu) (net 1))
 (segment (start 252.857 120.396) (end 251.333 121.92) (width 0.25) (layer F.Cu) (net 1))
 (segment (start 251.333 121.92) (end 242.189 121.92) (width 0.25) (layer F.Cu) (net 1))
 (segment (start 242.189 121.92) (end 240.538 120.269) (width 0.25) (layer F.Cu) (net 1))
 (segment (start 237.49 116.078) (end 237.617 116.078) (width 0.25) (layer F.Cu) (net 1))
 (segment (start 237.617 116.078) (end 240.538 118.999) (width 0.25) (layer F.Cu) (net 1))
 (segment (start 240.538 118.999) (end 240.538 120.269) (width 0.25) (layer F.Cu) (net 1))
 (segment (start 237.871 98.806) (end 240.792 98.806) (width 0.25) (layer F.Cu) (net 4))
 (segment (start 243.078 101.092) (end 243.078 109.093) (width 0.25) (layer F.Cu) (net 4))
 (segment (start 240.792 98.806) (end 243.078 101.092) (width 0.25) (layer F.Cu) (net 4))
 (segment (start 256.54 115.951) (end 256.54 112.268) (width 0.25) (layer F.Cu) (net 4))
 (segment (start 243.078 109.093) (end 243.078 120.269) (width 0.25) (layer F.Cu) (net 4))
 (segment (start 245.491 106.68) (end 243.078 109.093) (width 0.25) (layer F.Cu) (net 4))
 (segment (start 257.048 106.68) (end 245.491 106.68) (width 0.25) (layer F.Cu) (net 4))
 (segment (start 258.064 107.696) (end 257.048 106.68) (width 0.25) (layer F.Cu) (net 4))
 (segment (start 258.064 110.744) (end 258.064 107.696) (width 0.25) (layer F.Cu) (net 4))
 (segment (start 256.54 112.268) (end 258.064 110.744) (width 0.25) (layer F.Cu) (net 4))
 (segment (start 255.905 108.458) (end 253.619 108.458) (width 0.25) (layer F.Cu) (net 3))
 (segment (start 250.063 112.014) (end 250.063 119.888) (width 0.25) (layer F.Cu) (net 3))
 (segment (start 253.619 108.458) (end 250.063 112.014) (width 0.25) (layer F.Cu) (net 3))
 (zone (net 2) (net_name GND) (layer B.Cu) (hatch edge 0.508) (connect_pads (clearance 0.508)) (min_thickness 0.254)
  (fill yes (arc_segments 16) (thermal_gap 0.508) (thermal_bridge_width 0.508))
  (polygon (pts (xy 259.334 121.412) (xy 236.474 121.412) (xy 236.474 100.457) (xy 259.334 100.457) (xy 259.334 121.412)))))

